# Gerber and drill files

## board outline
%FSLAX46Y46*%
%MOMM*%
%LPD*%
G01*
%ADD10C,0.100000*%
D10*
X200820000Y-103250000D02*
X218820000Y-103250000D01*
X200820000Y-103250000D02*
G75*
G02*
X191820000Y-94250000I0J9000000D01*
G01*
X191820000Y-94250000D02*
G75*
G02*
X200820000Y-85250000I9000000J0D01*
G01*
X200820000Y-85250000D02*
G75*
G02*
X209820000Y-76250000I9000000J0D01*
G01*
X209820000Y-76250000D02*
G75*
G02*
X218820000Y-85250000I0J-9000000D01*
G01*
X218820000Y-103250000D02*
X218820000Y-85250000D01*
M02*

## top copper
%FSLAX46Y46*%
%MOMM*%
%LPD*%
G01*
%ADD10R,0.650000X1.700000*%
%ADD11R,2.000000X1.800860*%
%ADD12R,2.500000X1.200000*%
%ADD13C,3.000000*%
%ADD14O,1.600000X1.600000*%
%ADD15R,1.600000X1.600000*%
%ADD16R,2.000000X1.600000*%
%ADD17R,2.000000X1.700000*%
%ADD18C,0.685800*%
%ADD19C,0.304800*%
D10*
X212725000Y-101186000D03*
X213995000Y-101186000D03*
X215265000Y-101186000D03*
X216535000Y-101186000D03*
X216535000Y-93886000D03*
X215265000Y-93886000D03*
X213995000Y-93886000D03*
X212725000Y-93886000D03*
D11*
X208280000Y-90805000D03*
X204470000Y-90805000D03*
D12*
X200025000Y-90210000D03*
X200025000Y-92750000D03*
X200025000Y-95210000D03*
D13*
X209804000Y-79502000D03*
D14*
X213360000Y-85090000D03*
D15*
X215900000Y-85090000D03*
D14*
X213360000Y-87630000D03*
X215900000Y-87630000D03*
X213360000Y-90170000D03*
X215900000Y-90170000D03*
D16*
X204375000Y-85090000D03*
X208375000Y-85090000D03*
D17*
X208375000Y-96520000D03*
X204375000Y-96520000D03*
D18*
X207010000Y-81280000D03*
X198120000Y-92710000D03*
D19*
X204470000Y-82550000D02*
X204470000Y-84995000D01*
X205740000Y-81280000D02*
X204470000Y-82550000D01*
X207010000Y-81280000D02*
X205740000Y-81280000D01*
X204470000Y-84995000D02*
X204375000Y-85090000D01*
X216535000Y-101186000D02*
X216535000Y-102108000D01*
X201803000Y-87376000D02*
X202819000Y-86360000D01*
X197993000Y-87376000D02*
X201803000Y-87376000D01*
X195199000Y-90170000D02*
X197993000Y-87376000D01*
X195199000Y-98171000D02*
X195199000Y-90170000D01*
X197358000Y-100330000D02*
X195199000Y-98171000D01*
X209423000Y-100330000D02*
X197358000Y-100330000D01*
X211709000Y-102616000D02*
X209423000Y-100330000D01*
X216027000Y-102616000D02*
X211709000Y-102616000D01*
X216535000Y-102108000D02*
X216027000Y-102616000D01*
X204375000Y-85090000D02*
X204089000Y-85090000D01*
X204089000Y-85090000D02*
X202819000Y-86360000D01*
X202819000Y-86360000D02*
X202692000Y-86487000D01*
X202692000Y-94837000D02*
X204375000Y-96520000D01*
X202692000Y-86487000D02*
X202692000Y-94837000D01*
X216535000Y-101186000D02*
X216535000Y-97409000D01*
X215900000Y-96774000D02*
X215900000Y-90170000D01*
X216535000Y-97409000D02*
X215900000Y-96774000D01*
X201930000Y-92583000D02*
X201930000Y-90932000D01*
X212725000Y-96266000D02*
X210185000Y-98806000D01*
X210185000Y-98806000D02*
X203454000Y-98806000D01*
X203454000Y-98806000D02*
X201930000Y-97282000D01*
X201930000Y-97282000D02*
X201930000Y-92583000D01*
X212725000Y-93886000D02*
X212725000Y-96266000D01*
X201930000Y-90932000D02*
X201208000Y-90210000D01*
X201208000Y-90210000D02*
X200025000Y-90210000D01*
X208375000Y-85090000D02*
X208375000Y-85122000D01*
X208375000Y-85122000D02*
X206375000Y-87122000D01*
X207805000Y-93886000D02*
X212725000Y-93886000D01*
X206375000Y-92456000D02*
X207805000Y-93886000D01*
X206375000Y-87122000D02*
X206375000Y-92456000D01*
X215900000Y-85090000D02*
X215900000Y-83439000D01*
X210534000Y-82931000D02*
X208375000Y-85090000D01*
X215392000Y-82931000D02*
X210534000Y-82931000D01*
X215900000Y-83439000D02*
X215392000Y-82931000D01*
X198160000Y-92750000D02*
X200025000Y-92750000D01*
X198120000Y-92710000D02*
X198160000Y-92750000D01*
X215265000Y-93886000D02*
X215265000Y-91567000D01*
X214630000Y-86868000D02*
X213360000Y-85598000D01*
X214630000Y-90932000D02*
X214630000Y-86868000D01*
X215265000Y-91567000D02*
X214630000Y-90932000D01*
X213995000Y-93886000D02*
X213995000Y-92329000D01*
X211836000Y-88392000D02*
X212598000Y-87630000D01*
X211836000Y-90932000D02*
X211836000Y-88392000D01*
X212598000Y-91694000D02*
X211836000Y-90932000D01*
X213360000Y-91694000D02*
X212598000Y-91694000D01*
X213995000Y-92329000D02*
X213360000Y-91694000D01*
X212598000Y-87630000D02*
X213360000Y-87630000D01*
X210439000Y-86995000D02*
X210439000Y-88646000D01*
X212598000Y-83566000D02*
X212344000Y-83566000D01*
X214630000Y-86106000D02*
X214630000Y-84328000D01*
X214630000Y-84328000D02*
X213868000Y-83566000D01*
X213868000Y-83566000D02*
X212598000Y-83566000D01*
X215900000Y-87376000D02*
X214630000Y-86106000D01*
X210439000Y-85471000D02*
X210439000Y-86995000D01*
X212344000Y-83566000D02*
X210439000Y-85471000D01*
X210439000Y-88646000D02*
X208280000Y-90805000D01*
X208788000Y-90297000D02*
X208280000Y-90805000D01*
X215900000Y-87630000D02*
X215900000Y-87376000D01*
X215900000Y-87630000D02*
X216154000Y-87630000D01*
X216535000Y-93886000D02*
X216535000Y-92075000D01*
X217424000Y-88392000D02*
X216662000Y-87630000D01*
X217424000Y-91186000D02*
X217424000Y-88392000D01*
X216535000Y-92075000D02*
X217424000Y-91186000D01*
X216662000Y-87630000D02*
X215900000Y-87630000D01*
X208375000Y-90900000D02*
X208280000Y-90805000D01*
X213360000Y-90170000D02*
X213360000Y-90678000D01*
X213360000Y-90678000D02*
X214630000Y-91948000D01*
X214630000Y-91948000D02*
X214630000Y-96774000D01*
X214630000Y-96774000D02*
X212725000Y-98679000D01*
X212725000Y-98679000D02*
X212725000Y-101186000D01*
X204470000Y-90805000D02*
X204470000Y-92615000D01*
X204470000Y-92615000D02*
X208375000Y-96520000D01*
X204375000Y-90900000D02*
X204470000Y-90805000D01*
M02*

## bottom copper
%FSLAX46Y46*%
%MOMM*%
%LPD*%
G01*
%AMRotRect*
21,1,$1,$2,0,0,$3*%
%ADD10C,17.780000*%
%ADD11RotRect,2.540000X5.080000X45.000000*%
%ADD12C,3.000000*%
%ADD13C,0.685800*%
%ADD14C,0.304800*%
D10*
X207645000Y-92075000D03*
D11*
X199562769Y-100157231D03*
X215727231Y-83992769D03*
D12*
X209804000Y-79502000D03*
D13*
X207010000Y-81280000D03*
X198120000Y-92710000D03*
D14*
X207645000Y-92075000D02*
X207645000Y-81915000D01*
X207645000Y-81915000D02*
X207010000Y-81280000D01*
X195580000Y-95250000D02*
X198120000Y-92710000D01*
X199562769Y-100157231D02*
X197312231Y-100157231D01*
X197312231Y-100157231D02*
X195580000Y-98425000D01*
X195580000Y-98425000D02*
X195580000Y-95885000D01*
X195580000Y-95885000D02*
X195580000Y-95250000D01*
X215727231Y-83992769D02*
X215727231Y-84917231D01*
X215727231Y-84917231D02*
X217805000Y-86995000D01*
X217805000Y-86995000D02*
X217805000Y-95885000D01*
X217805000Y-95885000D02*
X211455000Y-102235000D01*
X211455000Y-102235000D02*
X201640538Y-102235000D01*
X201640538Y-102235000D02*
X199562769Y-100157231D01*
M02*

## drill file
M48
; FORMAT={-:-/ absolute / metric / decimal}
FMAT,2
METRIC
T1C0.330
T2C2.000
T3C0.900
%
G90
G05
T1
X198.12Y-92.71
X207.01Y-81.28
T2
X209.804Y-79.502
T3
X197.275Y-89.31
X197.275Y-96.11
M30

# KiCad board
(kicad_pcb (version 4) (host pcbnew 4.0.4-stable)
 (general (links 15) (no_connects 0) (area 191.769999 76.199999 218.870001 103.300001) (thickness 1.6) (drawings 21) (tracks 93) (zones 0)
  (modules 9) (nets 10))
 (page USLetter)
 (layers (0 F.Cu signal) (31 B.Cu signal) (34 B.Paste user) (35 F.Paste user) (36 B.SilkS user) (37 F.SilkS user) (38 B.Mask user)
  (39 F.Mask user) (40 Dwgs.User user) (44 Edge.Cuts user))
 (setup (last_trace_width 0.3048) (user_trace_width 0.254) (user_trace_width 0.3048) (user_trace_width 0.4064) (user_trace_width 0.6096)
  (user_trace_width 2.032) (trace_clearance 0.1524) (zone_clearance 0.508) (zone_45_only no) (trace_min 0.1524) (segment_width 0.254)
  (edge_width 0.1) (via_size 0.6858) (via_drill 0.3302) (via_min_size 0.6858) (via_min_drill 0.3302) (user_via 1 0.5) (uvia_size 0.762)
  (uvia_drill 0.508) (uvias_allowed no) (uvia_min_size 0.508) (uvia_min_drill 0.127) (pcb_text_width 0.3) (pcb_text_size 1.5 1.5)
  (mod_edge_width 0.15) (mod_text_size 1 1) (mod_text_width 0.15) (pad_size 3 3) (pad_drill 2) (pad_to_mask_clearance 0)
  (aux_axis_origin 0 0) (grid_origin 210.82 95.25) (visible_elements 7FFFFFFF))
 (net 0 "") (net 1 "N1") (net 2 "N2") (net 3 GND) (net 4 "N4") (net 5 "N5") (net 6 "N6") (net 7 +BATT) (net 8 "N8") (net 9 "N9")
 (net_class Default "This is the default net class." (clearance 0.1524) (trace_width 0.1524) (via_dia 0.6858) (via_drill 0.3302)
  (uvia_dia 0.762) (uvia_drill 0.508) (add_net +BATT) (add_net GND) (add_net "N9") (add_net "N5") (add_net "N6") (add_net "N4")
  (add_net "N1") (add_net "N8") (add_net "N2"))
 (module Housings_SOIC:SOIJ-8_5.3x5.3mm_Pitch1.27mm (layer F.Cu) (at 214.63 97.536 90)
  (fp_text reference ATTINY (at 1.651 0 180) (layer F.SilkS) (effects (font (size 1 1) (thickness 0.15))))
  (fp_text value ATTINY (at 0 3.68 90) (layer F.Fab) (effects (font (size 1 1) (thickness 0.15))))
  (pad 1 smd rect (at -3.65 -1.905 90) (size 1.7 0.65) (layers F.Cu F.Paste F.Mask) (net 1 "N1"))
  (pad 2 smd rect (at -3.65 -0.635 90) (size 1.7 0.65) (layers F.Cu F.Paste F.Mask) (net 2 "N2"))
  (pad 3 smd rect (at -3.65 0.635 90) (size 1.7 0.65) (layers F.Cu F.Paste F.Mask))
  (pad 4 smd rect (at -3.65 1.905 90) (size 1.7 0.65) (layers F.Cu F.Paste F.Mask) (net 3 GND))
  (pad 5 smd rect (at 3.65 1.905 90) (size 1.7 0.65) (layers F.Cu F.Paste F.Mask) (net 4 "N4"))
  (pad 6 smd rect (at 3.65 0.635 90) (size 1.7 0.65) (layers F.Cu F.Paste F.Mask) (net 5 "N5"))
  (pad 7 smd rect (at 3.65 -0.635 90) (size 1.7 0.65) (layers F.Cu F.Paste F.Mask) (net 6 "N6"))
  (pad 8 smd rect (at 3.65 -1.905 90) (size 1.7 0.65) (layers F.Cu F.Paste F.Mask) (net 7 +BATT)))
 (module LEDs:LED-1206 (layer F.Cu) (at 206.375 90.805)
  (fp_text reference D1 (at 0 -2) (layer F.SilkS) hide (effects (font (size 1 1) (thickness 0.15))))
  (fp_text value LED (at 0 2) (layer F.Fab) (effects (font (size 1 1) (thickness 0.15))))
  (pad 2 smd rect (at 1.905 0 180) (size 2 1.80086) (layers F.Cu F.Paste F.Mask) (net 4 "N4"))
  (pad 1 smd rect (at -1.905 0 180) (size 2 1.80086) (layers F.Cu F.Paste F.Mask) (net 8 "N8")))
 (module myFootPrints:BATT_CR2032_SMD (layer B.Cu) (at 207.645 92.075 45)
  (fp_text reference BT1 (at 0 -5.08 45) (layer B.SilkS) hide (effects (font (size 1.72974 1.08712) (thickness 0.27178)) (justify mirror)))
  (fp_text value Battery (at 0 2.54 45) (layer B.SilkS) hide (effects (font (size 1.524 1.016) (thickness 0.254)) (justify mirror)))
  (pad 2 smd circle (at 0 0 45) (size 17.78 17.78) (layers B.Cu B.Paste B.Mask) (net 3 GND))
  (pad 1 smd rect (at -11.43 0 45) (size 2.54 5.08) (layers B.Cu B.Paste B.Mask) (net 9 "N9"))
  (pad 1 smd rect (at 11.43 0 45) (size 2.54 5.08) (layers B.Cu B.Paste B.Mask) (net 9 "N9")))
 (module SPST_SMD (layer F.Cu) (at 200.025 92.71 270)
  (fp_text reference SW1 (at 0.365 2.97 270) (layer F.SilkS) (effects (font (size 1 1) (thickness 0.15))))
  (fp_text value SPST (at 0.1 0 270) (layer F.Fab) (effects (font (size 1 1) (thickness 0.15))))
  (pad "" np_thru_hole circle (at 3.4 2.75 270) (size 0.9 0.9) (drill 0.9) (layers *.Cu *.Mask))
  (pad 1 smd rect (at -2.5 0 270) (size 1.2 2.5) (layers F.Cu F.Paste F.Mask) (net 7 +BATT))
  (pad 2 smd rect (at 0.04 0 270) (size 1.2 2.5) (layers F.Cu F.Paste F.Mask) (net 9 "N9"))
  (pad 3 smd rect (at 2.5 0 270) (size 1.2 2.5) (layers F.Cu F.Paste F.Mask))
  (pad "" np_thru_hole circle (at -3.4 2.75 270) (size 0.9 0.9) (drill 0.9) (layers *.Cu *.Mask)))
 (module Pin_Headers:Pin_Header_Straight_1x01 (layer F.Cu) (at 209.804 79.502)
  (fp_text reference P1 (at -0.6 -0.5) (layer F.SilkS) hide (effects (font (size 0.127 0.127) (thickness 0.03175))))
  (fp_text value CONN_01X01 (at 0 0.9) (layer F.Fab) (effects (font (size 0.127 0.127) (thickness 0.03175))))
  (pad "" thru_hole circle (at 0 0) (size 3 3) (drill 2) (layers *.Cu *.Mask)))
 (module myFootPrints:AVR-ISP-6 (layer F.Cu) (at 213.36 85.09)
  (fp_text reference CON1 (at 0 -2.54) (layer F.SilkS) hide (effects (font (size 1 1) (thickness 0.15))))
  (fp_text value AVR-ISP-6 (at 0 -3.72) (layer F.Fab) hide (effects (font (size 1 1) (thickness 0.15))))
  (pad 1 smd oval (at 0 0) (size 1.6 1.6) (layers F.Cu F.Paste F.Mask) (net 5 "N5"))
  (pad 2 smd rect (at 2.54 0) (size 1.6 1.6) (layers F.Cu F.Paste F.Mask) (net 7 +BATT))
  (pad 3 smd oval (at 0 2.54) (size 1.6 1.6) (layers F.Cu F.Paste F.Mask) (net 6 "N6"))
  (pad 4 smd oval (at 2.54 2.54) (size 1.6 1.6) (layers F.Cu F.Paste F.Mask) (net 4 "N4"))
  (pad 5 smd oval (at 0 5.08) (size 1.6 1.6) (layers F.Cu F.Paste F.Mask) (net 1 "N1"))
  (pad 6 smd oval (at 2.54 5.08) (size 1.6 1.6) (layers F.Cu F.Paste F.Mask) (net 3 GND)))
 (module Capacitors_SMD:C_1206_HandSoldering (layer F.Cu) (at 206.375 85.09)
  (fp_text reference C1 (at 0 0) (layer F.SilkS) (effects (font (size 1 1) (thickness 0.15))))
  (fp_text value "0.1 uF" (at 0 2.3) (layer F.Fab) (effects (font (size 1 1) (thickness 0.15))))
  (pad 1 smd rect (at -2 0) (size 2 1.6) (layers F.Cu F.Paste F.Mask) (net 3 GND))
  (pad 2 smd rect (at 2 0) (size 2 1.6) (layers F.Cu F.Paste F.Mask) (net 7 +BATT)))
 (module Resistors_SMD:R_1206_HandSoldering (layer F.Cu) (at 206.375 96.52 180)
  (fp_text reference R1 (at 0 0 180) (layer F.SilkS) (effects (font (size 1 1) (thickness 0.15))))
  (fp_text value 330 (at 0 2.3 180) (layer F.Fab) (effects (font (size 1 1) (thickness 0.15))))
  (pad 1 smd rect (at -2 0 180) (size 2 1.7) (layers F.Cu F.Paste F.Mask) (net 8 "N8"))
  (pad 2 smd rect (at 2 0 180) (size 2 1.7) (layers F.Cu F.Paste F.Mask) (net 3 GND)))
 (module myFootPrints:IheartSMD (layer F.Cu) (at 203.835 100.33)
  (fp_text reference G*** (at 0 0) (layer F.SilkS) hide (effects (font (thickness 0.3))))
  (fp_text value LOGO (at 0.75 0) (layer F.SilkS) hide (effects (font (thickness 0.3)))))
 (gr_line (start 200.82 103.25) (end 218.82 103.25) (angle 90) (layer Edge.Cuts) (width 0.1))
 (gr_arc (start 200.82 94.25) (end 200.82 103.25) (angle 90) (layer Edge.Cuts) (width 0.1))
 (gr_arc (start 200.82 94.25) (end 191.82 94.25) (angle 90) (layer Edge.Cuts) (width 0.1))
 (gr_arc (start 209.82 85.25) (end 200.82 85.25) (angle 90) (layer Edge.Cuts) (width 0.1))
 (gr_arc (start 209.82 85.25) (end 209.82 76.25) (angle 90) (layer Edge.Cuts) (width 0.1))
 (gr_line (start 218.82 103.25) (end 218.82 85.25) (angle 90) (layer Edge.Cuts) (width 0.1))
 (segment (start 207.645 92.075) (end 207.645 81.915) (width 0.3048) (layer B.Cu) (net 3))
 (segment (start 204.47 82.55) (end 204.47 84.995) (width 0.3048) (layer F.Cu) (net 3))
 (segment (start 205.74 81.28) (end 204.47 82.55) (width 0.3048) (layer F.Cu) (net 3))
 (segment (start 207.01 81.28) (end 205.74 81.28) (width 0.3048) (layer F.Cu) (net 3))
 (via (at 207.01 81.28) (size 0.6858) (drill 0.3302) (layers F.Cu B.Cu) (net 3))
 (segment (start 207.645 81.915) (end 207.01 81.28) (width 0.3048) (layer B.Cu) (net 3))
 (segment (start 204.47 84.995) (end 204.375 85.09) (width 0.3048) (layer F.Cu) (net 3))
 (segment (start 216.535 101.186) (end 216.535 102.108) (width 0.3048) (layer F.Cu) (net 3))
 (segment (start 201.803 87.376) (end 202.819 86.36) (width 0.3048) (layer F.Cu) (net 3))
 (segment (start 197.993 87.376) (end 201.803 87.376) (width 0.3048) (layer F.Cu) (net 3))
 (segment (start 195.199 90.17) (end 197.993 87.376) (width 0.3048) (layer F.Cu) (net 3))
 (segment (start 195.199 98.171) (end 195.199 90.17) (width 0.3048) (layer F.Cu) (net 3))
 (segment (start 197.358 100.33) (end 195.199 98.171) (width 0.3048) (layer F.Cu) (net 3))
 (segment (start 209.423 100.33) (end 197.358 100.33) (width 0.3048) (layer F.Cu) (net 3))
 (segment (start 211.709 102.616) (end 209.423 100.33) (width 0.3048) (layer F.Cu) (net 3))
 (segment (start 216.027 102.616) (end 211.709 102.616) (width 0.3048) (layer F.Cu) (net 3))
 (segment (start 216.535 102.108) (end 216.027 102.616) (width 0.3048) (layer F.Cu) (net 3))
 (segment (start 204.375 85.09) (end 204.089 85.09) (width 0.3048) (layer F.Cu) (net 3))
 (segment (start 204.089 85.09) (end 202.819 86.36) (width 0.3048) (layer F.Cu) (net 3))
 (segment (start 202.819 86.36) (end 202.692 86.487) (width 0.3048) (layer F.Cu) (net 3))
 (segment (start 202.692 94.837) (end 204.375 96.52) (width 0.3048) (layer F.Cu) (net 3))
 (segment (start 202.692 86.487) (end 202.692 94.837) (width 0.3048) (layer F.Cu) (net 3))
 (segment (start 216.535 101.186) (end 216.535 97.409) (width 0.3048) (layer F.Cu) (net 3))
 (segment (start 215.9 96.774) (end 215.9 90.17) (width 0.3048) (layer F.Cu) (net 3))
 (segment (start 216.535 97.409) (end 215.9 96.774) (width 0.3048) (layer F.Cu) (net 3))
 (segment (start 201.93 92.583) (end 201.93 90.932) (width 0.3048) (layer F.Cu) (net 7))
 (segment (start 212.725 96.266) (end 210.185 98.806) (width 0.3048) (layer F.Cu) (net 7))
 (segment (start 210.185 98.806) (end 203.454 98.806) (width 0.3048) (layer F.Cu) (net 7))
 (segment (start 203.454 98.806) (end 201.93 97.282) (width 0.3048) (layer F.Cu) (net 7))
 (segment (start 201.93 97.282) (end 201.93 92.583) (width 0.3048) (layer F.Cu) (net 7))
 (segment (start 212.725 93.886) (end 212.725 96.266) (width 0.3048) (layer F.Cu) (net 7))
 (segment (start 201.93 90.932) (end 201.208 90.21) (width 0.3048) (layer F.Cu) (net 7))
 (segment (start 201.208 90.21) (end 200.025 90.21) (width 0.3048) (layer F.Cu) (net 7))
 (segment (start 208.375 85.09) (end 208.375 85.122) (width 0.3048) (layer F.Cu) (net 7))
 (segment (start 208.375 85.122) (end 206.375 87.122) (width 0.3048) (layer F.Cu) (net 7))
 (segment (start 207.805 93.886) (end 212.725 93.886) (width 0.3048) (layer F.Cu) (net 7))
 (segment (start 206.375 92.456) (end 207.805 93.886) (width 0.3048) (layer F.Cu) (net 7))
 (segment (start 206.375 87.122) (end 206.375 92.456) (width 0.3048) (layer F.Cu) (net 7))
 (segment (start 215.9 85.09) (end 215.9 83.439) (width 0.3048) (layer F.Cu) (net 7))
 (segment (start 210.534 82.931) (end 208.375 85.09) (width 0.3048) (layer F.Cu) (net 7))
 (segment (start 215.392 82.931) (end 210.534 82.931) (width 0.3048) (layer F.Cu) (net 7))
 (segment (start 215.9 83.439) (end 215.392 82.931) (width 0.3048) (layer F.Cu) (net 7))
 (segment (start 195.58 95.25) (end 198.12 92.71) (width 0.3048) (layer B.Cu) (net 9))
 (segment (start 198.16 92.75) (end 200.025 92.75) (width 0.3048) (layer F.Cu) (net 9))
 (via (at 198.12 92.71) (size 0.6858) (drill 0.3302) (layers F.Cu B.Cu) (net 9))
 (segment (start 198.12 92.71) (end 198.16 92.75) (width 0.3048) (layer F.Cu) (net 9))
 (segment (start 199.562769 100.157231) (end 197.312231 100.157231) (width 0.3048) (layer B.Cu) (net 9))
 (segment (start 197.312231 100.157231) (end 195.58 98.425) (width 0.3048) (layer B.Cu) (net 9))
 (segment (start 195.58 98.425) (end 195.58 95.885) (width 0.3048) (layer B.Cu) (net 9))
 (segment (start 195.58 95.885) (end 195.58 95.25) (width 0.3048) (layer B.Cu) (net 9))
 (segment (start 215.727231 83.992769) (end 215.727231 84.917231) (width 0.3048) (layer B.Cu) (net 9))
 (segment (start 215.727231 84.917231) (end 217.805 86.995) (width 0.3048) (layer B.Cu) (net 9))
 (segment (start 217.805 86.995) (end 217.805 95.885) (width 0.3048) (layer B.Cu) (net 9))
 (segment (start 217.805 95.885) (end 211.455 102.235) (width 0.3048) (layer B.Cu) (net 9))
 (segment (start 211.455 102.235) (end 201.640538 102.235) (width 0.3048) (layer B.Cu) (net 9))
 (segment (start 201.640538 102.235) (end 199.562769 100.157231) (width 0.3048) (layer B.Cu) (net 9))
 (segment (start 215.265 93.886) (end 215.265 91.567) (width 0.3048) (layer F.Cu) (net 5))
 (segment (start 214.63 86.868) (end 213.36 85.598) (width 0.3048) (layer F.Cu) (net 5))
 (segment (start 214.63 90.932) (end 214.63 86.868) (width 0.3048) (layer F.Cu) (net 5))
 (segment (start 215.265 91.567) (end 214.63 90.932) (width 0.3048) (layer F.Cu) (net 5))
 (segment (start 213.995 93.886) (end 213.995 92.329) (width 0.3048) (layer F.Cu) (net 6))
 (segment (start 211.836 88.392) (end 212.598 87.63) (width 0.3048) (layer F.Cu) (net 6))
 (segment (start 211.836 90.932) (end 211.836 88.392) (width 0.3048) (layer F.Cu) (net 6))
 (segment (start 212.598 91.694) (end 211.836 90.932) (width 0.3048) (layer F.Cu) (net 6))
 (segment (start 213.36 91.694) (end 212.598 91.694) (width 0.3048) (layer F.Cu) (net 6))
 (segment (start 213.995 92.329) (end 213.36 91.694) (width 0.3048) (layer F.Cu) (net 6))
 (segment (start 212.598 87.63) (end 213.36 87.63) (width 0.3048) (layer F.Cu) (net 6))
 (segment (start 210.439 86.995) (end 210.439 88.646) (width 0.3048) (layer F.Cu) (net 4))
 (segment (start 212.598 83.566) (end 212.344 83.566) (width 0.3048) (layer F.Cu) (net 4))
 (segment (start 214.63 86.106) (end 214.63 84.328) (width 0.3048) (layer F.Cu) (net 4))
 (segment (start 214.63 84.328) (end 213.868 83.566) (width 0.3048) (layer F.Cu) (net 4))
 (segment (start 213.868 83.566) (end 212.598 83.566) (width 0.3048) (layer F.Cu) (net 4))
 (segment (start 215.9 87.376) (end 214.63 86.106) (width 0.3048) (layer F.Cu) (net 4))
 (segment (start 210.439 85.471) (end 210.439 86.995) (width 0.3048) (layer F.Cu) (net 4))
 (segment (start 212.344 83.566) (end 210.439 85.471) (width 0.3048) (layer F.Cu) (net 4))
 (segment (start 210.439 88.646) (end 208.28 90.805) (width 0.3048) (layer F.Cu) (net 4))
 (segment (start 208.788 90.297) (end 208.28 90.805) (width 0.3048) (layer F.Cu) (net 4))
 (segment (start 215.9 87.63) (end 215.9 87.376) (width 0.3048) (layer F.Cu) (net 4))
 (segment (start 215.9 87.63) (end 216.154 87.63) (width 0.3048) (layer F.Cu) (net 4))
 (segment (start 216.535 93.886) (end 216.535 92.075) (width 0.3048) (layer F.Cu) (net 4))
 (segment (start 217.424 88.392) (end 216.662 87.63) (width 0.3048) (layer F.Cu) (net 4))
 (segment (start 217.424 91.186) (end 217.424 88.392) (width 0.3048) (layer F.Cu) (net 4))
 (segment (start 216.535 92.075) (end 217.424 91.186) (width 0.3048) (layer F.Cu) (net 4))
 (segment (start 216.662 87.63) (end 215.9 87.63) (width 0.3048) (layer F.Cu) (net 4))
 (segment (start 208.375 90.9) (end 208.28 90.805) (width 0.3048) (layer F.Cu) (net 4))
 (segment (start 213.36 90.17) (end 213.36 90.678) (width 0.3048) (layer F.Cu) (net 1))
 (segment (start 213.36 90.678) (end 214.63 91.948) (width 0.3048) (layer F.Cu) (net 1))
 (segment (start 214.63 91.948) (end 214.63 96.774) (width 0.3048) (layer F.Cu) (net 1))
 (segment (start 214.63 96.774) (end 212.725 98.679) (width 0.3048) (layer F.Cu) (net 1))
 (segment (start 212.725 98.679) (end 212.725 101.186) (width 0.3048) (layer F.Cu) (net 1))
 (segment (start 204.47 90.805) (end 204.47 92.615) (width 0.3048) (layer F.Cu) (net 8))
 (segment (start 204.47 92.615) (end 208.375 96.52) (width 0.3048) (layer F.Cu) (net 8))
 (segment (start 204.375 90.9) (end 204.47 90.805) (width 0.3048) (layer F.Cu) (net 8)))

